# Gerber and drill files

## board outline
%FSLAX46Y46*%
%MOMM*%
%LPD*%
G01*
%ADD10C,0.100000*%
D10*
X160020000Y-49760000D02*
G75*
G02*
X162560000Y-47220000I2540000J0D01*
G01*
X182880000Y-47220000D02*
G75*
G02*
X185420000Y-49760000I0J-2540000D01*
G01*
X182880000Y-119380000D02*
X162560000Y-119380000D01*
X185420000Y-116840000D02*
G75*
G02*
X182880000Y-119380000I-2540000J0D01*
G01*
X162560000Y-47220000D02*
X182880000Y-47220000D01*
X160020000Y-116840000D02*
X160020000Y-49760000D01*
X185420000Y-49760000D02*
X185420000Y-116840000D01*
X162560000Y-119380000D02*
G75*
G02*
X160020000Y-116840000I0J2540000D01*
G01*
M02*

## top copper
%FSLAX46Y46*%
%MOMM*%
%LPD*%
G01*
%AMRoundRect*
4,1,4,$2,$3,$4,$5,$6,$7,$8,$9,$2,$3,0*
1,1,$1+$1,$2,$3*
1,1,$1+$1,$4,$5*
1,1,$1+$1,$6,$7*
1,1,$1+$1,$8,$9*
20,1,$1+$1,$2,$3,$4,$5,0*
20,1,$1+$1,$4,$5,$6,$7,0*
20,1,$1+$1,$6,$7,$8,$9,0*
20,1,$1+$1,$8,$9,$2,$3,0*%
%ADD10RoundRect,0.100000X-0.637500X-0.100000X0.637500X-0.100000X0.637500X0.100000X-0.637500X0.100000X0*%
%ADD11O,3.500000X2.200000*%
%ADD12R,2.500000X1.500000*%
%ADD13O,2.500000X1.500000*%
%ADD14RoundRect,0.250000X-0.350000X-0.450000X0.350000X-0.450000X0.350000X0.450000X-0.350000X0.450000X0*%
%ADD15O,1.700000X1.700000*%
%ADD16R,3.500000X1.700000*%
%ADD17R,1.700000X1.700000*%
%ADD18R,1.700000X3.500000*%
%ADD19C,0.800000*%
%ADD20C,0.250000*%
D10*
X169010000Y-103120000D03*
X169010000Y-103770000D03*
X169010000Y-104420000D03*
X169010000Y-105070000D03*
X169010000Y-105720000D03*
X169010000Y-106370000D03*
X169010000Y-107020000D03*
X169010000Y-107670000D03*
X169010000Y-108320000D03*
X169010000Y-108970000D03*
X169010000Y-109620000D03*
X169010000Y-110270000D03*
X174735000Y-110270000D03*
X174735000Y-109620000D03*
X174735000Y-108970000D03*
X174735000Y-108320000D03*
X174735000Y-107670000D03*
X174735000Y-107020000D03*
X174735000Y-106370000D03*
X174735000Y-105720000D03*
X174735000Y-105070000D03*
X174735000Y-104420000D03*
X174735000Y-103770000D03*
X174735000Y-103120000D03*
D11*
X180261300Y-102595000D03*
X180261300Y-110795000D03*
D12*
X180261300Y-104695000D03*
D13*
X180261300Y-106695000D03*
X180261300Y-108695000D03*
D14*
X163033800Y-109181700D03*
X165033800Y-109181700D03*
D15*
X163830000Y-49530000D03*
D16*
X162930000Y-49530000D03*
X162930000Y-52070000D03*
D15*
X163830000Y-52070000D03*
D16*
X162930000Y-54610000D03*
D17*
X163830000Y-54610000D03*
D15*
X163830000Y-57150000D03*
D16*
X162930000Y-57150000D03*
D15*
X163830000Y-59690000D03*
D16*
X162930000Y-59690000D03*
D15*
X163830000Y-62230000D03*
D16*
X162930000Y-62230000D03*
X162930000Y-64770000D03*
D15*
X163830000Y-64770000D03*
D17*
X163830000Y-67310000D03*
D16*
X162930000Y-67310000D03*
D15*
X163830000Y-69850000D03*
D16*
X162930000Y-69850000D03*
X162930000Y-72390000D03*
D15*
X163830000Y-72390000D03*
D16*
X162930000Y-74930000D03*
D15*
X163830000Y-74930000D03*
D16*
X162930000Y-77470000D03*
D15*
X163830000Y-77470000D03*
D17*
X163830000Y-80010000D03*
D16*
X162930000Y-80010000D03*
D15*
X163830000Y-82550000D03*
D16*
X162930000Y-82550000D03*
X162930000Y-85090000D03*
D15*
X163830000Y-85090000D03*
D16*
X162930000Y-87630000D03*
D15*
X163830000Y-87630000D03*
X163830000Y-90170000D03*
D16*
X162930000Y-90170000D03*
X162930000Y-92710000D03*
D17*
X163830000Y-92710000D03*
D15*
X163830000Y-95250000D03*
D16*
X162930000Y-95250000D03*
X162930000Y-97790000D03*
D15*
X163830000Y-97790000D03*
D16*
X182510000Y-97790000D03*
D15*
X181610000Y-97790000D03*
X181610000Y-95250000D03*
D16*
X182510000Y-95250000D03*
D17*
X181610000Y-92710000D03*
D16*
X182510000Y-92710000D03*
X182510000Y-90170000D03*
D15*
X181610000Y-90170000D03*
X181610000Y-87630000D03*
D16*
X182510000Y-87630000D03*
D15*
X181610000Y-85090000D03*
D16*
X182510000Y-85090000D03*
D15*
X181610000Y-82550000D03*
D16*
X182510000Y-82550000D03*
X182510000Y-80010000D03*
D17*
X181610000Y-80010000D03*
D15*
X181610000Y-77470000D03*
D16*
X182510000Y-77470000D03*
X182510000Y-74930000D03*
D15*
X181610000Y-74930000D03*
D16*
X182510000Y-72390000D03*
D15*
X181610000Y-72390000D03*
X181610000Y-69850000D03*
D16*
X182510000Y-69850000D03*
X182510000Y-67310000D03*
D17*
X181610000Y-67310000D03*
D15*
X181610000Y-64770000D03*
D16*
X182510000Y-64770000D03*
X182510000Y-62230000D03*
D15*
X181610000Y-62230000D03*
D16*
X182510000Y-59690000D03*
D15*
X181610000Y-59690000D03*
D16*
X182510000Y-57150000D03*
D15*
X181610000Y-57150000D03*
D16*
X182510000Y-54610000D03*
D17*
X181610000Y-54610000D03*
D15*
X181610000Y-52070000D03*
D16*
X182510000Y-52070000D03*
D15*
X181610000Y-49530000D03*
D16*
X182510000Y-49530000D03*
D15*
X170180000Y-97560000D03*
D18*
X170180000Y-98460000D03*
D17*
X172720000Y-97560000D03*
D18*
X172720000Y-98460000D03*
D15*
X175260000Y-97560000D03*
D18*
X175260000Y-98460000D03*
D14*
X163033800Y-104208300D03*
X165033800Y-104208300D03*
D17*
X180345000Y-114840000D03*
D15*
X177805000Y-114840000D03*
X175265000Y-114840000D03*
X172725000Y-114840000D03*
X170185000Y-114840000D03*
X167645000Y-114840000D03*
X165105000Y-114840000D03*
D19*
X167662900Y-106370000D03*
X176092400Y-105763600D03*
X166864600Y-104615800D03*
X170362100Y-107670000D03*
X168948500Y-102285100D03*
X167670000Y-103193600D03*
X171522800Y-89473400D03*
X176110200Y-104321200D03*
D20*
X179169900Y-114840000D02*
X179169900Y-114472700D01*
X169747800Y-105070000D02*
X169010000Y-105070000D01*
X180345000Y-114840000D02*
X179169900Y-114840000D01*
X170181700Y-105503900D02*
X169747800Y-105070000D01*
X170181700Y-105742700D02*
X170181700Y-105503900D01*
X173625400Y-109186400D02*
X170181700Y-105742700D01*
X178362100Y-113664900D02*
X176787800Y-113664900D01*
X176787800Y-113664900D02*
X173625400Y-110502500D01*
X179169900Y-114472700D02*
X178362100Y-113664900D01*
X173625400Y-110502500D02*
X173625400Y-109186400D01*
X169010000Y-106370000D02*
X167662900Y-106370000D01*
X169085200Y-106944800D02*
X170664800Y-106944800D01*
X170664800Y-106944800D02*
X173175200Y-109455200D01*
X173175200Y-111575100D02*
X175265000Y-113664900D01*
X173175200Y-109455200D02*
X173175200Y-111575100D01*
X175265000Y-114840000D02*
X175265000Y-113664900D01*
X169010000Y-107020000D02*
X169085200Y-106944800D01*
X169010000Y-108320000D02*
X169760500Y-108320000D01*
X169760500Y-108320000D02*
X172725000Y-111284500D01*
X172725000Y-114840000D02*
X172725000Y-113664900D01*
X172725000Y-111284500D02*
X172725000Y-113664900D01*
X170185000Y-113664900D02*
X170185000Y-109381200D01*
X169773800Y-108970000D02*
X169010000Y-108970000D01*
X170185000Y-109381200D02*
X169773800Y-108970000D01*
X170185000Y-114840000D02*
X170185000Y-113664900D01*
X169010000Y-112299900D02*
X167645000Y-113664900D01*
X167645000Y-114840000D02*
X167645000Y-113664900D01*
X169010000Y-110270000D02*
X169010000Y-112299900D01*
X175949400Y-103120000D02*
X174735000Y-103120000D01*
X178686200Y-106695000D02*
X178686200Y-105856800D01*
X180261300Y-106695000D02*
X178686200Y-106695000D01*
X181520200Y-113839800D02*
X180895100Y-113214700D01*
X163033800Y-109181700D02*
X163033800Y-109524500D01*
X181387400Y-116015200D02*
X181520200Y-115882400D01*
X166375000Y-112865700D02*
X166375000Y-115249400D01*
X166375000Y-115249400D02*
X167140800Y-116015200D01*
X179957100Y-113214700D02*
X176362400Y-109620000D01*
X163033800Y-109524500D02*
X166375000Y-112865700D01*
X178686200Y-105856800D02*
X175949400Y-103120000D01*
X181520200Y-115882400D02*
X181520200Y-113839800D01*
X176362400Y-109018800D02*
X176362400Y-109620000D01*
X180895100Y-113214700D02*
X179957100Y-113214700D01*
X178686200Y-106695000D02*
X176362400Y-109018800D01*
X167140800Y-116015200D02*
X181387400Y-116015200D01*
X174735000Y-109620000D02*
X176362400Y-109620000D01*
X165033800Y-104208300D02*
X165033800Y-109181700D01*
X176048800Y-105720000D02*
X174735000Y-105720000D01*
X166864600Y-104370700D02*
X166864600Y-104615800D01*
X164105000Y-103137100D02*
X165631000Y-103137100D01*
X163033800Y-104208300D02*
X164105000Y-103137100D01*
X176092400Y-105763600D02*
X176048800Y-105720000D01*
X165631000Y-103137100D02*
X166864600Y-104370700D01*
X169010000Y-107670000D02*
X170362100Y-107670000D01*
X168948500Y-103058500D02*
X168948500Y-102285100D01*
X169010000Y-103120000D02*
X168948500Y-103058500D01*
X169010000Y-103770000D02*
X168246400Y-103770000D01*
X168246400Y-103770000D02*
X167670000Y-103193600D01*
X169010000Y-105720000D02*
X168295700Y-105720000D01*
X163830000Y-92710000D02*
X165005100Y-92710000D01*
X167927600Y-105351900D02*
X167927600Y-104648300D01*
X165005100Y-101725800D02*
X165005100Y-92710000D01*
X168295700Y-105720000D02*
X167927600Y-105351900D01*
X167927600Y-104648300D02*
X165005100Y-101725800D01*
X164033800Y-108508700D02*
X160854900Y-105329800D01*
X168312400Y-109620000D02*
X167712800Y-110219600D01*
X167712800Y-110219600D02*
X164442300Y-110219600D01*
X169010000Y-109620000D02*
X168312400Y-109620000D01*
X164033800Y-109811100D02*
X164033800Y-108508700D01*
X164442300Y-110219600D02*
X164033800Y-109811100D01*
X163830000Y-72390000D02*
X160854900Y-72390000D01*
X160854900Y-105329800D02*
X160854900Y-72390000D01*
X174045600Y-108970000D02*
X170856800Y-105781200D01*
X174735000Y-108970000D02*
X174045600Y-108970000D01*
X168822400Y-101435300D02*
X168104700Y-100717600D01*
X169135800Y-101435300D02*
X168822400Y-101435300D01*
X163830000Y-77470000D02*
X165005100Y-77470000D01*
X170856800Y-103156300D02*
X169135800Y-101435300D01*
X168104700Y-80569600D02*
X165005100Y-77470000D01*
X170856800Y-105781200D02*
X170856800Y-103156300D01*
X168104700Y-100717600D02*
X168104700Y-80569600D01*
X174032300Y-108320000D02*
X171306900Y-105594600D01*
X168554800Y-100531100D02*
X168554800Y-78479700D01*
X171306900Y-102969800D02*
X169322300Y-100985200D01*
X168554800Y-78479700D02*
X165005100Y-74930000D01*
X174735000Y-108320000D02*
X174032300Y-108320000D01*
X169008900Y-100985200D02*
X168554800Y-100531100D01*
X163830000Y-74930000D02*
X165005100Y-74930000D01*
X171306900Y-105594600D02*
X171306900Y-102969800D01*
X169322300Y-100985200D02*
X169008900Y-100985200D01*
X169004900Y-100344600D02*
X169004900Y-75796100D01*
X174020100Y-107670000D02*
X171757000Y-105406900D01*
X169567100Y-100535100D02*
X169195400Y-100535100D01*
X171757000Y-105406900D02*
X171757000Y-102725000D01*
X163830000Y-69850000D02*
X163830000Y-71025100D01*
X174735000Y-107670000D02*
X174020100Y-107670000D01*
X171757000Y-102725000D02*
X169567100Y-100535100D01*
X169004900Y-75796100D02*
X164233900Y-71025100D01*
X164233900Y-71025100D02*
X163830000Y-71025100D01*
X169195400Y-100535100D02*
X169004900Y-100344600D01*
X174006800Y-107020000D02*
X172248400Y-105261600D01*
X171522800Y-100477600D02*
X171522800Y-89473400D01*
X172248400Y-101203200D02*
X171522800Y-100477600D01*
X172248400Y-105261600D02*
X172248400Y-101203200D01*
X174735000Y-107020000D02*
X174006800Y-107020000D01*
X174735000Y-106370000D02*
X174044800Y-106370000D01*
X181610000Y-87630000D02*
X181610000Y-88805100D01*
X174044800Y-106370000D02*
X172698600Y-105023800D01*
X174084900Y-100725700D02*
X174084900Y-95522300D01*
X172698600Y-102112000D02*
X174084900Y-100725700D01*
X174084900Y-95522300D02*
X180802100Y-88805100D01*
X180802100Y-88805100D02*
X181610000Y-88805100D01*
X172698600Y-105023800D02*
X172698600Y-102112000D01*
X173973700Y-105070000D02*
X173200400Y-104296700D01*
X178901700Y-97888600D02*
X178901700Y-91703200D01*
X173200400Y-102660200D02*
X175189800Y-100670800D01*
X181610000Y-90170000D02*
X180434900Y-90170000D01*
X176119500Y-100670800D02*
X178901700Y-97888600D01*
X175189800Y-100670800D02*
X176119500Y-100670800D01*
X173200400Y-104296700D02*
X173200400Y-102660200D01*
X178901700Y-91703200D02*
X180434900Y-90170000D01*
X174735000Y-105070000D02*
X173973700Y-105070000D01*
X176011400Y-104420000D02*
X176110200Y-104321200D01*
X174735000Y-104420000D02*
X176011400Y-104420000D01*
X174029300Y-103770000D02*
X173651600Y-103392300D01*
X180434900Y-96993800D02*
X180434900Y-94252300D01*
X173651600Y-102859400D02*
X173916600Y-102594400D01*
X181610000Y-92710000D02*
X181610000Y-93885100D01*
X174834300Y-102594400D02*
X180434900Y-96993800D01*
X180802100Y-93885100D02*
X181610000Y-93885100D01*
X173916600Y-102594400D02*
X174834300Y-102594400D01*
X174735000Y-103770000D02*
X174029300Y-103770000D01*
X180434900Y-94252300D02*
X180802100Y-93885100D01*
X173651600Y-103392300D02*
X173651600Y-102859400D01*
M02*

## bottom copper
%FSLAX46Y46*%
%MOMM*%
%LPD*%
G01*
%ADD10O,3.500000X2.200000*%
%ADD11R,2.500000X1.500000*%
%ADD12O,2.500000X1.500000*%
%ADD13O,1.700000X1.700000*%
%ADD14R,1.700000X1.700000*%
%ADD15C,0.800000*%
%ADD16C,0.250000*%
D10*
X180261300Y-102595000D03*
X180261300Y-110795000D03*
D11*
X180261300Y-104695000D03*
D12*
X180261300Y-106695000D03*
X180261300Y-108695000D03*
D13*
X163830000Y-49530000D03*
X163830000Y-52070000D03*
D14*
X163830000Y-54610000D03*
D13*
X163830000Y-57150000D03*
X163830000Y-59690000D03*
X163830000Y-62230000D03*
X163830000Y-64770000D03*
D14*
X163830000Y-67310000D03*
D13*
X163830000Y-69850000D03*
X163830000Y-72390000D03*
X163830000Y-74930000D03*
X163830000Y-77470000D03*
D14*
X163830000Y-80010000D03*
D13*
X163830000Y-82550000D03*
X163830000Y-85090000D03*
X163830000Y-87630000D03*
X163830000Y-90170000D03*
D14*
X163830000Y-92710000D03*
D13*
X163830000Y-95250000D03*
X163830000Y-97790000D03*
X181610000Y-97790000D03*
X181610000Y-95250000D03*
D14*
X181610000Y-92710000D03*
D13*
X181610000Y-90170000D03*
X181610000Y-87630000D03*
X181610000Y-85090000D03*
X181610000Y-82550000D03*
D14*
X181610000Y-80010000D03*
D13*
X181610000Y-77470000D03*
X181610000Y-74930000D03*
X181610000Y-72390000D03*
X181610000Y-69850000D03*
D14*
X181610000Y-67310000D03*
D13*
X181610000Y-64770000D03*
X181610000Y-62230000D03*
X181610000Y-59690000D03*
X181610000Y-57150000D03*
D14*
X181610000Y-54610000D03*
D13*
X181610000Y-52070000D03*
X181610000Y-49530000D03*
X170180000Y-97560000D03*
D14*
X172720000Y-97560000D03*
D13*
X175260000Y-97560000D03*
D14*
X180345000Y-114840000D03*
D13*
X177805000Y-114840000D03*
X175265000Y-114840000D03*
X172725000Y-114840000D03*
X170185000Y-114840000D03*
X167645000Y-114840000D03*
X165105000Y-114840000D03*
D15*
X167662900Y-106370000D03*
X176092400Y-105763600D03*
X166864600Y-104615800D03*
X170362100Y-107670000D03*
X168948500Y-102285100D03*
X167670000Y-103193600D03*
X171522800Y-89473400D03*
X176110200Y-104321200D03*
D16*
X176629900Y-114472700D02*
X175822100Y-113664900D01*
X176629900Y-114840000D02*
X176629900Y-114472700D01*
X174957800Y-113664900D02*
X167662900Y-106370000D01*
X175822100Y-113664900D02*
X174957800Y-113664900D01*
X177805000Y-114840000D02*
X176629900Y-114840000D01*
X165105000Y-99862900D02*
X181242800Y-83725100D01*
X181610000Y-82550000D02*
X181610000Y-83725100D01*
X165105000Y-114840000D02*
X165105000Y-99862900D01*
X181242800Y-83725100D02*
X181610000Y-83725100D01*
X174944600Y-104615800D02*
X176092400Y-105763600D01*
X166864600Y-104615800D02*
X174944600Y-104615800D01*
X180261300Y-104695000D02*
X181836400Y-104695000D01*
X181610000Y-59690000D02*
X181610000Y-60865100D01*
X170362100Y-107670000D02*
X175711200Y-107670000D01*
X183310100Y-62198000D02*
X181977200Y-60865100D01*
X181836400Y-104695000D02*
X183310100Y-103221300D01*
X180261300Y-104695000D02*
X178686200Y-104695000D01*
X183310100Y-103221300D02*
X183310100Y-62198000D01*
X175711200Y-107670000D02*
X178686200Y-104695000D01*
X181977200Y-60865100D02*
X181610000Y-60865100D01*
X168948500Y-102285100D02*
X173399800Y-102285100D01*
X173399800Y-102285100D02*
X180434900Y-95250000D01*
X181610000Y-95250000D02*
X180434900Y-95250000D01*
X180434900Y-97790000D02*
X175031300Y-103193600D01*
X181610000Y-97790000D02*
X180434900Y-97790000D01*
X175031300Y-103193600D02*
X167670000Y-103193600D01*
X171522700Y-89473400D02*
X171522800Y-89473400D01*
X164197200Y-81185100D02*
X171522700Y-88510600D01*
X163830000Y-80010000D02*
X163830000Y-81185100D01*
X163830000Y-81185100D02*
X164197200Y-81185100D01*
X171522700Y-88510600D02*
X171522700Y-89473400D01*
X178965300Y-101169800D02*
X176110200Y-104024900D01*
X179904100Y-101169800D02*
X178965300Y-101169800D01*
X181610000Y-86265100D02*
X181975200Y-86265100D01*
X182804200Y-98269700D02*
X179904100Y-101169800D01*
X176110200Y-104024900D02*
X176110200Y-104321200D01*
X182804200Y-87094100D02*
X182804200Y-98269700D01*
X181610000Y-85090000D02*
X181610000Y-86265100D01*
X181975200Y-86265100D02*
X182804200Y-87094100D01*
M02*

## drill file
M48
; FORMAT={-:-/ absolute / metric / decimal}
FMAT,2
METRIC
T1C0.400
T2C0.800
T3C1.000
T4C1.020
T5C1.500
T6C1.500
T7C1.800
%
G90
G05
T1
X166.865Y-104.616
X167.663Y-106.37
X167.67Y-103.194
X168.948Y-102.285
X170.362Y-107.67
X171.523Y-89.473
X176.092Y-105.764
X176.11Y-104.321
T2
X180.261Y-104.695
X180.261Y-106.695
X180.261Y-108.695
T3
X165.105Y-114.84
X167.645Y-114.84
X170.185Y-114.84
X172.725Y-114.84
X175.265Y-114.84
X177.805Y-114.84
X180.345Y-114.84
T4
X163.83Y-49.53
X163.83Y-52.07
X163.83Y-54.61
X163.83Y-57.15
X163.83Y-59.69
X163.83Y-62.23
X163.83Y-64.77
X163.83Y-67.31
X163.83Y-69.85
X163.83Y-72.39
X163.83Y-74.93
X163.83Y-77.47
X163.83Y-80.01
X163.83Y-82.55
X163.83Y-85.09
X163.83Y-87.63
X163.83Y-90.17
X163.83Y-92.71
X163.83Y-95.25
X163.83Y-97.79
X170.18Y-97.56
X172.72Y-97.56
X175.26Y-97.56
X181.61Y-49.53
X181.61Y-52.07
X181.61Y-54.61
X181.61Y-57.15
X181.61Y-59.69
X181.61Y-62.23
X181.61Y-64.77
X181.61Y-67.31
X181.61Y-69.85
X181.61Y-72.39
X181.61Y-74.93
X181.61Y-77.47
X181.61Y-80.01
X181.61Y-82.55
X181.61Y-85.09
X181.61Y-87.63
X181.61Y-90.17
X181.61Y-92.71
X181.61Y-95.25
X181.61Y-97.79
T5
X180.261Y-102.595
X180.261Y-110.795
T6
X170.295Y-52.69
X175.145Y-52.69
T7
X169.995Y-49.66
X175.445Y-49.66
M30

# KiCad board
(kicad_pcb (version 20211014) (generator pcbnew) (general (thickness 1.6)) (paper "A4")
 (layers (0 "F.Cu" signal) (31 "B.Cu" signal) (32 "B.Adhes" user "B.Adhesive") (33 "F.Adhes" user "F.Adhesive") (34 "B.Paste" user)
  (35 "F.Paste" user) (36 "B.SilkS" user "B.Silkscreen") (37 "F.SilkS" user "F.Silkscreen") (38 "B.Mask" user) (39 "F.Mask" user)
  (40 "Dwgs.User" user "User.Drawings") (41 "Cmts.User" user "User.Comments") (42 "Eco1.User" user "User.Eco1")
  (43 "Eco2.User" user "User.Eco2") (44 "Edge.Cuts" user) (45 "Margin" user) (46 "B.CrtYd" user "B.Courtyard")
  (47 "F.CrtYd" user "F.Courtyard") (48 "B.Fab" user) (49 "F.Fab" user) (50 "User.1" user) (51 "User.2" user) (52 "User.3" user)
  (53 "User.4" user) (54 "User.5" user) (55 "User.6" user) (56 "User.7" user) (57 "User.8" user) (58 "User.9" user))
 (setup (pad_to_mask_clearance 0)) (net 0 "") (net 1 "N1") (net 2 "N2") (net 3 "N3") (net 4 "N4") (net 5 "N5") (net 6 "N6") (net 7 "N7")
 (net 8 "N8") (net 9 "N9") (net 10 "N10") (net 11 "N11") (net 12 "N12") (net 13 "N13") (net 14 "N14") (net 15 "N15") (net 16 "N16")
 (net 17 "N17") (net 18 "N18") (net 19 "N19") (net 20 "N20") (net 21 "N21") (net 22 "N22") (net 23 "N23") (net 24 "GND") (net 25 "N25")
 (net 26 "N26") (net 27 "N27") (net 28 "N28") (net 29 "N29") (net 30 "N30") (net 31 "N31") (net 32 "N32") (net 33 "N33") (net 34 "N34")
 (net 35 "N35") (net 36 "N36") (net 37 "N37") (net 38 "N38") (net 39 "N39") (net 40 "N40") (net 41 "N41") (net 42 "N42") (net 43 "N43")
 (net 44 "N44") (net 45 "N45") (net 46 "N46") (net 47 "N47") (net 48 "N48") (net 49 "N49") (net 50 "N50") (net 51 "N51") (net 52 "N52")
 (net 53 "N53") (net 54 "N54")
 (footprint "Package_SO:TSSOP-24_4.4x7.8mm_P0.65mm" (layer "F.Cu") (at 171.8725 106.695)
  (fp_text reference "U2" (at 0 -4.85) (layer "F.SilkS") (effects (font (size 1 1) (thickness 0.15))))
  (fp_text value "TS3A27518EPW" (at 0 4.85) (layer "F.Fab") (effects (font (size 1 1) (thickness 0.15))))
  (pad "1" smd roundrect (at -2.8625 -3.575) (size 1.475 0.4) (layers "F.Cu" "F.Paste" "F.Mask") (roundrect_rratio 0.25) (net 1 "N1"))
  (pad "2" smd roundrect (at -2.8625 -2.925) (size 1.475 0.4) (layers "F.Cu" "F.Paste" "F.Mask") (roundrect_rratio 0.25) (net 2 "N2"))
  (pad "3" smd roundrect (at -2.8625 -2.275) (size 1.475 0.4) (layers "F.Cu" "F.Paste" "F.Mask") (roundrect_rratio 0.25) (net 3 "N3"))
  (pad "4" smd roundrect (at -2.8625 -1.625) (size 1.475 0.4) (layers "F.Cu" "F.Paste" "F.Mask") (roundrect_rratio 0.25) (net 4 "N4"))
  (pad "5" smd roundrect (at -2.8625 -0.975) (size 1.475 0.4) (layers "F.Cu" "F.Paste" "F.Mask") (roundrect_rratio 0.25) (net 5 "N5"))
  (pad "6" smd roundrect (at -2.8625 -0.325) (size 1.475 0.4) (layers "F.Cu" "F.Paste" "F.Mask") (roundrect_rratio 0.25) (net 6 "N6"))
  (pad "7" smd roundrect (at -2.8625 0.325) (size 1.475 0.4) (layers "F.Cu" "F.Paste" "F.Mask") (roundrect_rratio 0.25) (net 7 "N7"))
  (pad "8" smd roundrect (at -2.8625 0.975) (size 1.475 0.4) (layers "F.Cu" "F.Paste" "F.Mask") (roundrect_rratio 0.25) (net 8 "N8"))
  (pad "9" smd roundrect (at -2.8625 1.625) (size 1.475 0.4) (layers "F.Cu" "F.Paste" "F.Mask") (roundrect_rratio 0.25) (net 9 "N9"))
  (pad "10" smd roundrect (at -2.8625 2.275) (size 1.475 0.4) (layers "F.Cu" "F.Paste" "F.Mask") (roundrect_rratio 0.25) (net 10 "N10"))
  (pad "11" smd roundrect (at -2.8625 2.925) (size 1.475 0.4) (layers "F.Cu" "F.Paste" "F.Mask") (roundrect_rratio 0.25) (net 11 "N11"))
  (pad "12" smd roundrect (at -2.8625 3.575) (size 1.475 0.4) (layers "F.Cu" "F.Paste" "F.Mask") (roundrect_rratio 0.25) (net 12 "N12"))
  (pad "13" smd roundrect (at 2.8625 3.575) (size 1.475 0.4) (layers "F.Cu" "F.Paste" "F.Mask") (roundrect_rratio 0.25) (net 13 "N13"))
  (pad "14" smd roundrect (at 2.8625 2.925) (size 1.475 0.4) (layers "F.Cu" "F.Paste" "F.Mask") (roundrect_rratio 0.25) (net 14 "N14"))
  (pad "15" smd roundrect (at 2.8625 2.275) (size 1.475 0.4) (layers "F.Cu" "F.Paste" "F.Mask") (roundrect_rratio 0.25) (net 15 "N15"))
  (pad "16" smd roundrect (at 2.8625 1.625) (size 1.475 0.4) (layers "F.Cu" "F.Paste" "F.Mask") (roundrect_rratio 0.25) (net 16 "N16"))
  (pad "17" smd roundrect (at 2.8625 0.975) (size 1.475 0.4) (layers "F.Cu" "F.Paste" "F.Mask") (roundrect_rratio 0.25) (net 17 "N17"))
  (pad "18" smd roundrect (at 2.8625 0.325) (size 1.475 0.4) (layers "F.Cu" "F.Paste" "F.Mask") (roundrect_rratio 0.25) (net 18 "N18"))
  (pad "19" smd roundrect (at 2.8625 -0.325) (size 1.475 0.4) (layers "F.Cu" "F.Paste" "F.Mask") (roundrect_rratio 0.25) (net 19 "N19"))
  (pad "20" smd roundrect (at 2.8625 -0.975) (size 1.475 0.4) (layers "F.Cu" "F.Paste" "F.Mask") (roundrect_rratio 0.25) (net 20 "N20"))
  (pad "21" smd roundrect (at 2.8625 -1.625) (size 1.475 0.4) (layers "F.Cu" "F.Paste" "F.Mask") (roundrect_rratio 0.25) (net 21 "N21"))
  (pad "22" smd roundrect (at 2.8625 -2.275) (size 1.475 0.4) (layers "F.Cu" "F.Paste" "F.Mask") (roundrect_rratio 0.25) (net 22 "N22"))
  (pad "23" smd roundrect (at 2.8625 -2.925) (size 1.475 0.4) (layers "F.Cu" "F.Paste" "F.Mask") (roundrect_rratio 0.25) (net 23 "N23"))
  (pad "24" smd roundrect (at 2.8625 -3.575) (size 1.475 0.4) (layers "F.Cu" "F.Paste" "F.Mask") (roundrect_rratio 0.25) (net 14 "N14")))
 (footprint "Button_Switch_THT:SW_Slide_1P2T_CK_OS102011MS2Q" (layer "F.Cu") (at 180.2613 104.695 -90)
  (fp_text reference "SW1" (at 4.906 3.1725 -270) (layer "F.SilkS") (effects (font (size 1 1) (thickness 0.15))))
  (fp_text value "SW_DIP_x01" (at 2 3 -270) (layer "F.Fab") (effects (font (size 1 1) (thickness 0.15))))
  (pad "" thru_hole oval (at -2.1 0 270) (size 2.2 3.5) (drill 1.5) (layers *.Cu *.Mask))
  (pad "" thru_hole oval (at 6.1 0 270) (size 2.2 3.5) (drill 1.5) (layers *.Cu *.Mask))
  (pad "1" thru_hole rect (at 0 0 270) (size 1.5 2.5) (drill 0.8) (layers *.Cu *.Mask) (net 8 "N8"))
  (pad "2" thru_hole oval (at 2 0 270) (size 1.5 2.5) (drill 0.8) (layers *.Cu *.Mask) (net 14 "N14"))
  (pad "3" thru_hole oval (at 4 0 270) (size 1.5 2.5) (drill 0.8) (layers *.Cu *.Mask)))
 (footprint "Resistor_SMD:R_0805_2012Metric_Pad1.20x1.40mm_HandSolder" (layer "F.Cu") (at 164.0338 109.1817)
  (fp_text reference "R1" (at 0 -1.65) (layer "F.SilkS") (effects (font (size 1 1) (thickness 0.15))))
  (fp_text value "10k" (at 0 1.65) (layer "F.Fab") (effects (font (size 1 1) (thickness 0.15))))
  (pad "1" smd roundrect (at -1 0) (size 1.2 1.4) (layers "F.Cu" "F.Paste" "F.Mask") (roundrect_rratio 0.208333) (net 14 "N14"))
  (pad "2" smd roundrect (at 1 0) (size 1.2 1.4) (layers "F.Cu" "F.Paste" "F.Mask") (roundrect_rratio 0.208333) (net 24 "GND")))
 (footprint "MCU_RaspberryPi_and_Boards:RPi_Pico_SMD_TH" (layer "F.Cu") (at 172.72 73.66)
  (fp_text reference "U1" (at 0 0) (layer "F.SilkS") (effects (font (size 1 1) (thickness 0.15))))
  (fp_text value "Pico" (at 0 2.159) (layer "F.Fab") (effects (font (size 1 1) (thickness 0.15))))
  (pad "" np_thru_hole oval (at 2.425 -20.97) (size 1.5 1.5) (drill 1.5) (layers *.Cu *.Mask))
  (pad "" np_thru_hole oval (at 2.725 -24) (size 1.8 1.8) (drill 1.8) (layers *.Cu *.Mask))
  (pad "" np_thru_hole oval (at -2.725 -24) (size 1.8 1.8) (drill 1.8) (layers *.Cu *.Mask))
  (pad "" np_thru_hole oval (at -2.425 -20.97) (size 1.5 1.5) (drill 1.5) (layers *.Cu *.Mask))
  (pad "1" thru_hole oval (at -8.89 -24.13) (size 1.7 1.7) (drill 1.02) (layers *.Cu *.Mask) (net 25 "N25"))
  (pad "1" smd rect (at -8.89 -24.13) (size 3.5 1.7) (drill (offset -0.9 0)) (layers "F.Cu" "F.Mask") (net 25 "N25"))
  (pad "2" smd rect (at -8.89 -21.59) (size 3.5 1.7) (drill (offset -0.9 0)) (layers "F.Cu" "F.Mask") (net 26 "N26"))
  (pad "2" thru_hole oval (at -8.89 -21.59) (size 1.7 1.7) (drill 1.02) (layers *.Cu *.Mask) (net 26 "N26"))
  (pad "3" smd rect (at -8.89 -19.05) (size 3.5 1.7) (drill (offset -0.9 0)) (layers "F.Cu" "F.Mask") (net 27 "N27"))
  (pad "3" thru_hole rect (at -8.89 -19.05) (size 1.7 1.7) (drill 1.02) (layers *.Cu *.Mask) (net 27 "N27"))
  (pad "4" thru_hole oval (at -8.89 -16.51) (size 1.7 1.7) (drill 1.02) (layers *.Cu *.Mask) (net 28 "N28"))
  (pad "4" smd rect (at -8.89 -16.51) (size 3.5 1.7) (drill (offset -0.9 0)) (layers "F.Cu" "F.Mask") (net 28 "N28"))
  (pad "5" thru_hole oval (at -8.89 -13.97) (size 1.7 1.7) (drill 1.02) (layers *.Cu *.Mask) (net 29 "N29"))
  (pad "5" smd rect (at -8.89 -13.97) (size 3.5 1.7) (drill (offset -0.9 0)) (layers "F.Cu" "F.Mask") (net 29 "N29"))
  (pad "6" thru_hole oval (at -8.89 -11.43) (size 1.7 1.7) (drill 1.02) (layers *.Cu *.Mask) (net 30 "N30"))
  (pad "6" smd rect (at -8.89 -11.43) (size 3.5 1.7) (drill (offset -0.9 0)) (layers "F.Cu" "F.Mask") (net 30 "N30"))
  (pad "7" smd rect (at -8.89 -8.89) (size 3.5 1.7) (drill (offset -0.9 0)) (layers "F.Cu" "F.Mask") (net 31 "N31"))
  (pad "7" thru_hole oval (at -8.89 -8.89) (size 1.7 1.7) (drill 1.02) (layers *.Cu *.Mask) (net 31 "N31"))
  (pad "8" thru_hole rect (at -8.89 -6.35) (size 1.7 1.7) (drill 1.02) (layers *.Cu *.Mask) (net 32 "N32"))
  (pad "8" smd rect (at -8.89 -6.35) (size 3.5 1.7) (drill (offset -0.9 0)) (layers "F.Cu" "F.Mask") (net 32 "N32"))
  (pad "9" thru_hole oval (at -8.89 -3.81) (size 1.7 1.7) (drill 1.02) (layers *.Cu *.Mask) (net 17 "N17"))
  (pad "9" smd rect (at -8.89 -3.81) (size 3.5 1.7) (drill (offset -0.9 0)) (layers "F.Cu" "F.Mask") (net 17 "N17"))
  (pad "10" smd rect (at -8.89 -1.27) (size 3.5 1.7) (drill (offset -0.9 0)) (layers "F.Cu" "F.Mask") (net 11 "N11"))
  (pad "10" thru_hole oval (at -8.89 -1.27) (size 1.7 1.7) (drill 1.02) (layers *.Cu *.Mask) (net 11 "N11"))
  (pad "11" smd rect (at -8.89 1.27) (size 3.5 1.7) (drill (offset -0.9 0)) (layers "F.Cu" "F.Mask") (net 16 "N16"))
  (pad "11" thru_hole oval (at -8.89 1.27) (size 1.7 1.7) (drill 1.02) (layers *.Cu *.Mask) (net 16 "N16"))
  (pad "12" smd rect (at -8.89 3.81) (size 3.5 1.7) (drill (offset -0.9 0)) (layers "F.Cu" "F.Mask") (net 15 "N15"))
  (pad "12" thru_hole oval (at -8.89 3.81) (size 1.7 1.7) (drill 1.02) (layers *.Cu *.Mask) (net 15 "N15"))
  (pad "13" thru_hole rect (at -8.89 6.35) (size 1.7 1.7) (drill 1.02) (layers *.Cu *.Mask) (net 18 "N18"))
  (pad "13" smd rect (at -8.89 6.35) (size 3.5 1.7) (drill (offset -0.9 0)) (layers "F.Cu" "F.Mask") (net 18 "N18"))
  (pad "14" thru_hole oval (at -8.89 8.89) (size 1.7 1.7) (drill 1.02) (layers *.Cu *.Mask) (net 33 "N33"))
  (pad "14" smd rect (at -8.89 8.89) (size 3.5 1.7) (drill (offset -0.9 0)) (layers "F.Cu" "F.Mask") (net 33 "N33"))
  (pad "15" smd rect (at -8.89 11.43) (size 3.5 1.7) (drill (offset -0.9 0)) (layers "F.Cu" "F.Mask") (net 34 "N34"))
  (pad "15" thru_hole oval (at -8.89 11.43) (size 1.7 1.7) (drill 1.02) (layers *.Cu *.Mask) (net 34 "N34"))
  (pad "16" smd rect (at -8.89 13.97) (size 3.5 1.7) (drill (offset -0.9 0)) (layers "F.Cu" "F.Mask") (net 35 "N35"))
  (pad "16" thru_hole oval (at -8.89 13.97) (size 1.7 1.7) (drill 1.02) (layers *.Cu *.Mask) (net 35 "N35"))
  (pad "17" thru_hole oval (at -8.89 16.51) (size 1.7 1.7) (drill 1.02) (layers *.Cu *.Mask) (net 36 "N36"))
  (pad "17" smd rect (at -8.89 16.51) (size 3.5 1.7) (drill (offset -0.9 0)) (layers "F.Cu" "F.Mask") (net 36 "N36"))
  (pad "18" smd rect (at -8.89 19.05) (size 3.5 1.7) (drill (offset -0.9 0)) (layers "F.Cu" "F.Mask") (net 5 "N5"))
  (pad "18" thru_hole rect (at -8.89 19.05) (size 1.7 1.7) (drill 1.02) (layers *.Cu *.Mask) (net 5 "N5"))
  (pad "19" thru_hole oval (at -8.89 21.59) (size 1.7 1.7) (drill 1.02) (layers *.Cu *.Mask) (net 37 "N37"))
  (pad "19" smd rect (at -8.89 21.59) (size 3.5 1.7) (drill (offset -0.9 0)) (layers "F.Cu" "F.Mask") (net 37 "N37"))
  (pad "20" smd rect (at -8.89 24.13) (size 3.5 1.7) (drill (offset -0.9 0)) (layers "F.Cu" "F.Mask") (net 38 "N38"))
  (pad "20" thru_hole oval (at -8.89 24.13) (size 1.7 1.7) (drill 1.02) (layers *.Cu *.Mask) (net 38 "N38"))
  (pad "21" smd rect (at 8.89 24.13) (size 3.5 1.7) (drill (offset 0.9 0)) (layers "F.Cu" "F.Mask") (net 2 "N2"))
  (pad "21" thru_hole oval (at 8.89 24.13) (size 1.7 1.7) (drill 1.02) (layers *.Cu *.Mask) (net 2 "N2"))
  (pad "22" thru_hole oval (at 8.89 21.59) (size 1.7 1.7) (drill 1.02) (layers *.Cu *.Mask) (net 1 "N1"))
  (pad "22" smd rect (at 8.89 21.59) (size 3.5 1.7) (drill (offset 0.9 0)) (layers "F.Cu" "F.Mask") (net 1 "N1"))
  (pad "23" thru_hole rect (at 8.89 19.05) (size 1.7 1.7) (drill 1.02) (layers *.Cu *.Mask) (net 23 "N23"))
  (pad "23" smd rect (at 8.89 19.05) (size 3.5 1.7) (drill (offset 0.9 0)) (layers "F.Cu" "F.Mask") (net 23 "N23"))
  (pad "24" smd rect (at 8.89 16.51) (size 3.5 1.7) (drill (offset 0.9 0)) (layers "F.Cu" "F.Mask") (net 21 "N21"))
  (pad "24" thru_hole oval (at 8.89 16.51) (size 1.7 1.7) (drill 1.02) (layers *.Cu *.Mask) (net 21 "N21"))
  (pad "25" thru_hole oval (at 8.89 13.97) (size 1.7 1.7) (drill 1.02) (layers *.Cu *.Mask) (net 19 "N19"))
  (pad "25" smd rect (at 8.89 13.97) (size 3.5 1.7) (drill (offset 0.9 0)) (layers "F.Cu" "F.Mask") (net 19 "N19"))
  (pad "26" thru_hole oval (at 8.89 11.43) (size 1.7 1.7) (drill 1.02) (layers *.Cu *.Mask) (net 22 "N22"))
  (pad "26" smd rect (at 8.89 11.43) (size 3.5 1.7) (drill (offset 0.9 0)) (layers "F.Cu" "F.Mask") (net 22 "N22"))
  (pad "27" thru_hole oval (at 8.89 8.89) (size 1.7 1.7) (drill 1.02) (layers *.Cu *.Mask) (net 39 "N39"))
  (pad "27" smd rect (at 8.89 8.89) (size 3.5 1.7) (drill (offset 0.9 0)) (layers "F.Cu" "F.Mask") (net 39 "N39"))
  (pad "28" smd rect (at 8.89 6.35) (size 3.5 1.7) (drill (offset 0.9 0)) (layers "F.Cu" "F.Mask") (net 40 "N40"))
  (pad "28" thru_hole rect (at 8.89 6.35) (size 1.7 1.7) (drill 1.02) (layers *.Cu *.Mask) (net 40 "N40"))
  (pad "29" thru_hole oval (at 8.89 3.81) (size 1.7 1.7) (drill 1.02) (layers *.Cu *.Mask) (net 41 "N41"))
  (pad "29" smd rect (at 8.89 3.81) (size 3.5 1.7) (drill (offset 0.9 0)) (layers "F.Cu" "F.Mask") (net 41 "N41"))
  (pad "30" smd rect (at 8.89 1.27) (size 3.5 1.7) (drill (offset 0.9 0)) (layers "F.Cu" "F.Mask") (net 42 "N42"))
  (pad "30" thru_hole oval (at 8.89 1.27) (size 1.7 1.7) (drill 1.02) (layers *.Cu *.Mask) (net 42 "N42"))
  (pad "31" smd rect (at 8.89 -1.27) (size 3.5 1.7) (drill (offset 0.9 0)) (layers "F.Cu" "F.Mask") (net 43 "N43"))
  (pad "31" thru_hole oval (at 8.89 -1.27) (size 1.7 1.7) (drill 1.02) (layers *.Cu *.Mask) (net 43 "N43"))
  (pad "32" thru_hole oval (at 8.89 -3.81) (size 1.7 1.7) (drill 1.02) (layers *.Cu *.Mask) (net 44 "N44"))
  (pad "32" smd rect (at 8.89 -3.81) (size 3.5 1.7) (drill (offset 0.9 0)) (layers "F.Cu" "F.Mask") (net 44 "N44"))
  (pad "33" smd rect (at 8.89 -6.35) (size 3.5 1.7) (drill (offset 0.9 0)) (layers "F.Cu" "F.Mask") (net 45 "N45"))
  (pad "33" thru_hole rect (at 8.89 -6.35) (size 1.7 1.7) (drill 1.02) (layers *.Cu *.Mask) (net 45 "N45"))
  (pad "34" thru_hole oval (at 8.89 -8.89) (size 1.7 1.7) (drill 1.02) (layers *.Cu *.Mask) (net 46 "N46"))
  (pad "34" smd rect (at 8.89 -8.89) (size 3.5 1.7) (drill (offset 0.9 0)) (layers "F.Cu" "F.Mask") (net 46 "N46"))
  (pad "35" smd rect (at 8.89 -11.43) (size 3.5 1.7) (drill (offset 0.9 0)) (layers "F.Cu" "F.Mask") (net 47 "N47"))
  (pad "35" thru_hole oval (at 8.89 -11.43) (size 1.7 1.7) (drill 1.02) (layers *.Cu *.Mask) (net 47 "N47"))
  (pad "36" smd rect (at 8.89 -13.97) (size 3.5 1.7) (drill (offset 0.9 0)) (layers "F.Cu" "F.Mask") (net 8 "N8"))
  (pad "36" thru_hole oval (at 8.89 -13.97) (size 1.7 1.7) (drill 1.02) (layers *.Cu *.Mask) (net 8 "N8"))
  (pad "37" smd rect (at 8.89 -16.51) (size 3.5 1.7) (drill (offset 0.9 0)) (layers "F.Cu" "F.Mask") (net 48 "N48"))
  (pad "37" thru_hole oval (at 8.89 -16.51) (size 1.7 1.7) (drill 1.02) (layers *.Cu *.Mask) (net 48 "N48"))
  (pad "38" smd rect (at 8.89 -19.05) (size 3.5 1.7) (drill (offset 0.9 0)) (layers "F.Cu" "F.Mask") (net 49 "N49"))
  (pad "38" thru_hole rect (at 8.89 -19.05) (size 1.7 1.7) (drill 1.02) (layers *.Cu *.Mask) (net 49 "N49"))
  (pad "39" thru_hole oval (at 8.89 -21.59) (size 1.7 1.7) (drill 1.02) (layers *.Cu *.Mask) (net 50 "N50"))
  (pad "39" smd rect (at 8.89 -21.59) (size 3.5 1.7) (drill (offset 0.9 0)) (layers "F.Cu" "F.Mask") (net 50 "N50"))
  (pad "40" thru_hole oval (at 8.89 -24.13) (size 1.7 1.7) (drill 1.02) (layers *.Cu *.Mask) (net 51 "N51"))
  (pad "40" smd rect (at 8.89 -24.13) (size 3.5 1.7) (drill (offset 0.9 0)) (layers "F.Cu" "F.Mask") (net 51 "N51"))
  (pad "41" thru_hole oval (at -2.54 23.9) (size 1.7 1.7) (drill 1.02) (layers *.Cu *.Mask) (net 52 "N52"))
  (pad "41" smd rect (at -2.54 23.9 90) (size 3.5 1.7) (drill (offset -0.9 0)) (layers "F.Cu" "F.Mask") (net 52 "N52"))
  (pad "42" thru_hole rect (at 0 23.9) (size 1.7 1.7) (drill 1.02) (layers *.Cu *.Mask) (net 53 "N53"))
  (pad "42" smd rect (at 0 23.9 90) (size 3.5 1.7) (drill (offset -0.9 0)) (layers "F.Cu" "F.Mask") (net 53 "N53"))
  (pad "43" thru_hole oval (at 2.54 23.9) (size 1.7 1.7) (drill 1.02) (layers *.Cu *.Mask) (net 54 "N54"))
  (pad "43" smd rect (at 2.54 23.9 90) (size 3.5 1.7) (drill (offset -0.9 0)) (layers "F.Cu" "F.Mask") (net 54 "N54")))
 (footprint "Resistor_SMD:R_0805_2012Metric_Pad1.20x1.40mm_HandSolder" (layer "F.Cu") (at 164.0338 104.2083)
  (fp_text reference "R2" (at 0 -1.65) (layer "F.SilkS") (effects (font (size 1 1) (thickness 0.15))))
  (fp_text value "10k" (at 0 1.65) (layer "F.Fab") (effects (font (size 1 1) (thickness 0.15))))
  (pad "1" smd roundrect (at -1 0) (size 1.2 1.4) (layers "F.Cu" "F.Paste" "F.Mask") (roundrect_rratio 0.208333) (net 20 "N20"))
  (pad "2" smd roundrect (at 1 0) (size 1.2 1.4) (layers "F.Cu" "F.Paste" "F.Mask") (roundrect_rratio 0.208333) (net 24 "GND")))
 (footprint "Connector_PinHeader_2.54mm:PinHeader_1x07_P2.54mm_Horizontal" (layer "F.Cu") (at 180.345 114.84 -90)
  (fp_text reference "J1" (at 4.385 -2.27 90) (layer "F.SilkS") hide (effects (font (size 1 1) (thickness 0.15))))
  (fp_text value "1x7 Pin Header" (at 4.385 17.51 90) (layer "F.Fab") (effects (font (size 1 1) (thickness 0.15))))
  (pad "1" thru_hole rect (at 0 0 270) (size 1.7 1.7) (drill 1) (layers *.Cu *.Mask) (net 4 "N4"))
  (pad "2" thru_hole oval (at 0 2.54 270) (size 1.7 1.7) (drill 1) (layers *.Cu *.Mask) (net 6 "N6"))
  (pad "3" thru_hole oval (at 0 5.08 270) (size 1.7 1.7) (drill 1) (layers *.Cu *.Mask) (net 7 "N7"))
  (pad "4" thru_hole oval (at 0 7.62 270) (size 1.7 1.7) (drill 1) (layers *.Cu *.Mask) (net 9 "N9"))
  (pad "5" thru_hole oval (at 0 10.16 270) (size 1.7 1.7) (drill 1) (layers *.Cu *.Mask) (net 10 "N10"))
  (pad "6" thru_hole oval (at 0 12.7 270) (size 1.7 1.7) (drill 1) (layers *.Cu *.Mask) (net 12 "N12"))
  (pad "7" thru_hole oval (at 0 15.24 270) (size 1.7 1.7) (drill 1) (layers *.Cu *.Mask) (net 39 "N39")))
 (gr_arc (start 160.02 49.76) (mid 160.763949 47.963949) (end 162.56 47.22) (layer "Edge.Cuts") (width 0.1))
 (gr_arc (start 182.88 47.22) (mid 184.676051 47.963949) (end 185.42 49.76) (layer "Edge.Cuts") (width 0.1))
 (gr_line (start 182.88 119.38) (end 162.56 119.38) (layer "Edge.Cuts") (width 0.1))
 (gr_arc (start 185.42 116.84) (mid 184.676051 118.636051) (end 182.88 119.38) (layer "Edge.Cuts") (width 0.1))
 (gr_line (start 162.56 47.22) (end 182.88 47.22) (layer "Edge.Cuts") (width 0.1))
 (gr_line (start 160.02 116.84) (end 160.02 49.76) (layer "Edge.Cuts") (width 0.1))
 (gr_line (start 185.42 49.76) (end 185.42 116.84) (layer "Edge.Cuts") (width 0.1))
 (gr_arc (start 162.56 119.38) (mid 160.763949 118.636051) (end 160.02 116.84) (layer "Edge.Cuts") (width 0.1))
 (segment (start 179.1699 114.84) (end 179.1699 114.4727) (width 0.25) (layer "F.Cu") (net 4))
 (segment (start 169.7478 105.07) (end 169.01 105.07) (width 0.25) (layer "F.Cu") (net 4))
 (segment (start 180.345 114.84) (end 179.1699 114.84) (width 0.25) (layer "F.Cu") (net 4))
 (segment (start 170.1817 105.5039) (end 169.7478 105.07) (width 0.25) (layer "F.Cu") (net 4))
 (segment (start 170.1817 105.7427) (end 170.1817 105.5039) (width 0.25) (layer "F.Cu") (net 4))
 (segment (start 173.6254 109.1864) (end 170.1817 105.7427) (width 0.25) (layer "F.Cu") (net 4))
 (segment (start 178.3621 113.6649) (end 176.7878 113.6649) (width 0.25) (layer "F.Cu") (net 4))
 (segment (start 176.7878 113.6649) (end 173.6254 110.5025) (width 0.25) (layer "F.Cu") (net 4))
 (segment (start 179.1699 114.4727) (end 178.3621 113.6649) (width 0.25) (layer "F.Cu") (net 4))
 (segment (start 173.6254 110.5025) (end 173.6254 109.1864) (width 0.25) (layer "F.Cu") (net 4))
 (segment (start 169.01 106.37) (end 167.6629 106.37) (width 0.25) (layer "F.Cu") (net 6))
 (via (at 167.6629 106.37) (size 0.8) (drill 0.4) (layers "F.Cu" "B.Cu") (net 6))
 (segment (start 176.6299 114.4727) (end 175.8221 113.6649) (width 0.25) (layer "B.Cu") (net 6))
 (segment (start 176.6299 114.84) (end 176.6299 114.4727) (width 0.25) (layer "B.Cu") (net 6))
 (segment (start 174.9578 113.6649) (end 167.6629 106.37) (width 0.25) (layer "B.Cu") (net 6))
 (segment (start 175.8221 113.6649) (end 174.9578 113.6649) (width 0.25) (layer "B.Cu") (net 6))
 (segment (start 177.805 114.84) (end 176.6299 114.84) (width 0.25) (layer "B.Cu") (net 6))
 (segment (start 169.0852 106.9448) (end 170.6648 106.9448) (width 0.25) (layer "F.Cu") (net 7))
 (segment (start 170.6648 106.9448) (end 173.1752 109.4552) (width 0.25) (layer "F.Cu") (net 7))
 (segment (start 173.1752 111.5751) (end 175.265 113.6649) (width 0.25) (layer "F.Cu") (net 7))
 (segment (start 173.1752 109.4552) (end 173.1752 111.5751) (width 0.25) (layer "F.Cu") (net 7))
 (segment (start 175.265 114.84) (end 175.265 113.6649) (width 0.25) (layer "F.Cu") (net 7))
 (segment (start 169.01 107.02) (end 169.0852 106.9448) (width 0.25) (layer "F.Cu") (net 7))
 (segment (start 169.01 108.32) (end 169.7605 108.32) (width 0.25) (layer "F.Cu") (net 9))
 (segment (start 169.7605 108.32) (end 172.725 111.2845) (width 0.25) (layer "F.Cu") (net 9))
 (segment (start 172.725 114.84) (end 172.725 113.6649) (width 0.25) (layer "F.Cu") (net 9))
 (segment (start 172.725 111.2845) (end 172.725 113.6649) (width 0.25) (layer "F.Cu") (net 9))
 (segment (start 170.185 113.6649) (end 170.185 109.3812) (width 0.25) (layer "F.Cu") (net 10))
 (segment (start 169.7738 108.97) (end 169.01 108.97) (width 0.25) (layer "F.Cu") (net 10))
 (segment (start 170.185 109.3812) (end 169.7738 108.97) (width 0.25) (layer "F.Cu") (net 10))
 (segment (start 170.185 114.84) (end 170.185 113.6649) (width 0.25) (layer "F.Cu") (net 10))
 (segment (start 169.01 112.2999) (end 167.645 113.6649) (width 0.25) (layer "F.Cu") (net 12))
 (segment (start 167.645 114.84) (end 167.645 113.6649) (width 0.25) (layer "F.Cu") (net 12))
 (segment (start 169.01 110.27) (end 169.01 112.2999) (width 0.25) (layer "F.Cu") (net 12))
 (segment (start 165.105 99.8629) (end 181.2428 83.7251) (width 0.25) (layer "B.Cu") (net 39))
 (segment (start 181.61 82.55) (end 181.61 83.7251) (width 0.25) (layer "B.Cu") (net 39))
 (segment (start 165.105 114.84) (end 165.105 99.8629) (width 0.25) (layer "B.Cu") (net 39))
 (segment (start 181.2428 83.7251) (end 181.61 83.7251) (width 0.25) (layer "B.Cu") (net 39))
 (segment (start 175.9494 103.12) (end 174.735 103.12) (width 0.25) (layer "F.Cu") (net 14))
 (segment (start 178.6862 106.695) (end 178.6862 105.8568) (width 0.25) (layer "F.Cu") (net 14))
 (segment (start 180.2613 106.695) (end 178.6862 106.695) (width 0.25) (layer "F.Cu") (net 14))
 (segment (start 181.5202 113.8398) (end 180.8951 113.2147) (width 0.25) (layer "F.Cu") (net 14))
 (segment (start 163.0338 109.1817) (end 163.0338 109.5245) (width 0.25) (layer "F.Cu") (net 14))
 (segment (start 181.3874 116.0152) (end 181.5202 115.8824) (width 0.25) (layer "F.Cu") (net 14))
 (segment (start 166.375 112.8657) (end 166.375 115.2494) (width 0.25) (layer "F.Cu") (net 14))
 (segment (start 166.375 115.2494) (end 167.1408 116.0152) (width 0.25) (layer "F.Cu") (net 14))
 (segment (start 179.9571 113.2147) (end 176.3624 109.62) (width 0.25) (layer "F.Cu") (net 14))
 (segment (start 163.0338 109.5245) (end 166.375 112.8657) (width 0.25) (layer "F.Cu") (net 14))
 (segment (start 178.6862 105.8568) (end 175.9494 103.12) (width 0.25) (layer "F.Cu") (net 14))
 (segment (start 181.5202 115.8824) (end 181.5202 113.8398) (width 0.25) (layer "F.Cu") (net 14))
 (segment (start 176.3624 109.0188) (end 176.3624 109.62) (width 0.25) (layer "F.Cu") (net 14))
 (segment (start 180.8951 113.2147) (end 179.9571 113.2147) (width 0.25) (layer "F.Cu") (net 14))
 (segment (start 178.6862 106.695) (end 176.3624 109.0188) (width 0.25) (layer "F.Cu") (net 14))
 (segment (start 167.1408 116.0152) (end 181.3874 116.0152) (width 0.25) (layer "F.Cu") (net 14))
 (segment (start 174.735 109.62) (end 176.3624 109.62) (width 0.25) (layer "F.Cu") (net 14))
 (segment (start 165.0338 104.2083) (end 165.0338 109.1817) (width 0.25) (layer "F.Cu") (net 24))
 (segment (start 176.0488 105.72) (end 174.735 105.72) (width 0.25) (layer "F.Cu") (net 20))
 (segment (start 166.8646 104.3707) (end 166.8646 104.6158) (width 0.25) (layer "F.Cu") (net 20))
 (segment (start 164.105 103.1371) (end 165.631 103.1371) (width 0.25) (layer "F.Cu") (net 20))
 (segment (start 163.0338 104.2083) (end 164.105 103.1371) (width 0.25) (layer "F.Cu") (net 20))
 (segment (start 176.0924 105.7636) (end 176.0488 105.72) (width 0.25) (layer "F.Cu") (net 20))
 (segment (start 165.631 103.1371) (end 166.8646 104.3707) (width 0.25) (layer "F.Cu") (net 20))
 (via (at 176.0924 105.7636) (size 0.8) (drill 0.4) (layers "F.Cu" "B.Cu") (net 20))
 (via (at 166.8646 104.6158) (size 0.8) (drill 0.4) (layers "F.Cu" "B.Cu") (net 20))
 (segment (start 174.9446 104.6158) (end 176.0924 105.7636) (width 0.25) (layer "B.Cu") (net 20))
 (segment (start 166.8646 104.6158) (end 174.9446 104.6158) (width 0.25) (layer "B.Cu") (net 20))
 (segment (start 169.01 107.67) (end 170.3621 107.67) (width 0.25) (layer "F.Cu") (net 8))
 (via (at 170.3621 107.67) (size 0.8) (drill 0.4) (layers "F.Cu" "B.Cu") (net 8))
 (segment (start 180.2613 104.695) (end 181.8364 104.695) (width 0.25) (layer "B.Cu") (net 8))
 (segment (start 181.61 59.69) (end 181.61 60.8651) (width 0.25) (layer "B.Cu") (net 8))
 (segment (start 170.3621 107.67) (end 175.7112 107.67) (width 0.25) (layer "B.Cu") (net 8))
 (segment (start 183.3101 62.198) (end 181.9772 60.8651) (width 0.25) (layer "B.Cu") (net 8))
 (segment (start 181.8364 104.695) (end 183.3101 103.2213) (width 0.25) (layer "B.Cu") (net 8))
 (segment (start 180.2613 104.695) (end 178.6862 104.695) (width 0.25) (layer "B.Cu") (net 8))
 (segment (start 183.3101 103.2213) (end 183.3101 62.198) (width 0.25) (layer "B.Cu") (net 8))
 (segment (start 175.7112 107.67) (end 178.6862 104.695) (width 0.25) (layer "B.Cu") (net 8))
 (segment (start 181.9772 60.8651) (end 181.61 60.8651) (width 0.25) (layer "B.Cu") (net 8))
 (segment (start 168.9485 103.0585) (end 168.9485 102.2851) (width 0.25) (layer "F.Cu") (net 1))
 (segment (start 169.01 103.12) (end 168.9485 103.0585) (width 0.25) (layer "F.Cu") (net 1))
 (via (at 168.9485 102.2851) (size 0.8) (drill 0.4) (layers "F.Cu" "B.Cu") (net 1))
 (segment (start 168.9485 102.2851) (end 173.3998 102.2851) (width 0.25) (layer "B.Cu") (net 1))
 (segment (start 173.3998 102.2851) (end 180.4349 95.25) (width 0.25) (layer "B.Cu") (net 1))
 (segment (start 181.61 95.25) (end 180.4349 95.25) (width 0.25) (layer "B.Cu") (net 1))
 (segment (start 169.01 103.77) (end 168.2464 103.77) (width 0.25) (layer "F.Cu") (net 2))
 (segment (start 168.2464 103.77) (end 167.67 103.1936) (width 0.25) (layer "F.Cu") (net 2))
 (via (at 167.67 103.1936) (size 0.8) (drill 0.4) (layers "F.Cu" "B.Cu") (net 2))
 (segment (start 180.4349 97.79) (end 175.0313 103.1936) (width 0.25) (layer "B.Cu") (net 2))
 (segment (start 181.61 97.79) (end 180.4349 97.79) (width 0.25) (layer "B.Cu") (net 2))
 (segment (start 175.0313 103.1936) (end 167.67 103.1936) (width 0.25) (layer "B.Cu") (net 2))
 (segment (start 169.01 105.72) (end 168.2957 105.72) (width 0.25) (layer "F.Cu") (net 5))
 (segment (start 163.83 92.71) (end 165.0051 92.71) (width 0.25) (layer "F.Cu") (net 5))
 (segment (start 167.9276 105.3519) (end 167.9276 104.6483) (width 0.25) (layer "F.Cu") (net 5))
 (segment (start 165.0051 101.7258) (end 165.0051 92.71) (width 0.25) (layer "F.Cu") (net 5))
 (segment (start 168.2957 105.72) (end 167.9276 105.3519) (width 0.25) (layer "F.Cu") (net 5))
 (segment (start 167.9276 104.6483) (end 165.0051 101.7258) (width 0.25) (layer "F.Cu") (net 5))
 (segment (start 164.0338 108.5087) (end 160.8549 105.3298) (width 0.25) (layer "F.Cu") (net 11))
 (segment (start 168.3124 109.62) (end 167.7128 110.2196) (width 0.25) (layer "F.Cu") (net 11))
 (segment (start 167.7128 110.2196) (end 164.4423 110.2196) (width 0.25) (layer "F.Cu") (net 11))
 (segment (start 169.01 109.62) (end 168.3124 109.62) (width 0.25) (layer "F.Cu") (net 11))
 (segment (start 164.0338 109.8111) (end 164.0338 108.5087) (width 0.25) (layer "F.Cu") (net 11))
 (segment (start 164.4423 110.2196) (end 164.0338 109.8111) (width 0.25) (layer "F.Cu") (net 11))
 (segment (start 163.83 72.39) (end 160.8549 72.39) (width 0.25) (layer "F.Cu") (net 11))
 (segment (start 160.8549 105.3298) (end 160.8549 72.39) (width 0.25) (layer "F.Cu") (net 11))
 (segment (start 174.0456 108.97) (end 170.8568 105.7812) (width 0.25) (layer "F.Cu") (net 15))
 (segment (start 174.735 108.97) (end 174.0456 108.97) (width 0.25) (layer "F.Cu") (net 15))
 (segment (start 168.8224 101.4353) (end 168.1047 100.7176) (width 0.25) (layer "F.Cu") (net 15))
 (segment (start 169.1358 101.4353) (end 168.8224 101.4353) (width 0.25) (layer "F.Cu") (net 15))
 (segment (start 163.83 77.47) (end 165.0051 77.47) (width 0.25) (layer "F.Cu") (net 15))
 (segment (start 170.8568 103.1563) (end 169.1358 101.4353) (width 0.25) (layer "F.Cu") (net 15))
 (segment (start 168.1047 80.5696) (end 165.0051 77.47) (width 0.25) (layer "F.Cu") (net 15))
 (segment (start 170.8568 105.7812) (end 170.8568 103.1563) (width 0.25) (layer "F.Cu") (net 15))
 (segment (start 168.1047 100.7176) (end 168.1047 80.5696) (width 0.25) (layer "F.Cu") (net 15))
 (segment (start 174.0323 108.32) (end 171.3069 105.5946) (width 0.25) (layer "F.Cu") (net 16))
 (segment (start 168.5548 100.5311) (end 168.5548 78.4797) (width 0.25) (layer "F.Cu") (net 16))
 (segment (start 171.3069 102.9698) (end 169.3223 100.9852) (width 0.25) (layer "F.Cu") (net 16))
 (segment (start 168.5548 78.4797) (end 165.0051 74.93) (width 0.25) (layer "F.Cu") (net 16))
 (segment (start 174.735 108.32) (end 174.0323 108.32) (width 0.25) (layer "F.Cu") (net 16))
 (segment (start 169.0089 100.9852) (end 168.5548 100.5311) (width 0.25) (layer "F.Cu") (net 16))
 (segment (start 163.83 74.93) (end 165.0051 74.93) (width 0.25) (layer "F.Cu") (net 16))
 (segment (start 171.3069 105.5946) (end 171.3069 102.9698) (width 0.25) (layer "F.Cu") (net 16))
 (segment (start 169.3223 100.9852) (end 169.0089 100.9852) (width 0.25) (layer "F.Cu") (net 16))
 (segment (start 169.0049 100.3446) (end 169.0049 75.7961) (width 0.25) (layer "F.Cu") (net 17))
 (segment (start 174.0201 107.67) (end 171.757 105.4069) (width 0.25) (layer "F.Cu") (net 17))
 (segment (start 169.5671 100.5351) (end 169.1954 100.5351) (width 0.25) (layer "F.Cu") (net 17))
 (segment (start 171.757 105.4069) (end 171.757 102.725) (width 0.25) (layer "F.Cu") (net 17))
 (segment (start 163.83 69.85) (end 163.83 71.0251) (width 0.25) (layer "F.Cu") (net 17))
 (segment (start 174.735 107.67) (end 174.0201 107.67) (width 0.25) (layer "F.Cu") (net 17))
 (segment (start 171.757 102.725) (end 169.5671 100.5351) (width 0.25) (layer "F.Cu") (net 17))
 (segment (start 169.0049 75.7961) (end 164.2339 71.0251) (width 0.25) (layer "F.Cu") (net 17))
 (segment (start 164.2339 71.0251) (end 163.83 71.0251) (width 0.25) (layer "F.Cu") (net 17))
 (segment (start 169.1954 100.5351) (end 169.0049 100.3446) (width 0.25) (layer "F.Cu") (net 17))
 (segment (start 174.0068 107.02) (end 172.2484 105.2616) (width 0.25) (layer "F.Cu") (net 18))
 (segment (start 171.5228 100.4776) (end 171.5228 89.4734) (width 0.25) (layer "F.Cu") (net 18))
 (segment (start 172.2484 101.2032) (end 171.5228 100.4776) (width 0.25) (layer "F.Cu") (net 18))
 (segment (start 172.2484 105.2616) (end 172.2484 101.2032) (width 0.25) (layer "F.Cu") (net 18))
 (segment (start 174.735 107.02) (end 174.0068 107.02) (width 0.25) (layer "F.Cu") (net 18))
 (via (at 171.5228 89.4734) (size 0.8) (drill 0.4) (layers "F.Cu" "B.Cu") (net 18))
 (segment (start 171.5227 89.4734) (end 171.5228 89.4734) (width 0.25) (layer "B.Cu") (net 18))
 (segment (start 164.1972 81.1851) (end 171.5227 88.5106) (width 0.25) (layer "B.Cu") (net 18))
 (segment (start 163.83 80.01) (end 163.83 81.1851) (width 0.25) (layer "B.Cu") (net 18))
 (segment (start 163.83 81.1851) (end 164.1972 81.1851) (width 0.25) (layer "B.Cu") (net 18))
 (segment (start 171.5227 88.5106) (end 171.5227 89.4734) (width 0.25) (layer "B.Cu") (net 18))
 (segment (start 174.735 106.37) (end 174.0448 106.37) (width 0.25) (layer "F.Cu") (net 19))
 (segment (start 181.61 87.63) (end 181.61 88.8051) (width 0.25) (layer "F.Cu") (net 19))
 (segment (start 174.0448 106.37) (end 172.6986 105.0238) (width 0.25) (layer "F.Cu") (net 19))
 (segment (start 174.0849 100.7257) (end 174.0849 95.5223) (width 0.25) (layer "F.Cu") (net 19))
 (segment (start 172.6986 102.112) (end 174.0849 100.7257) (width 0.25) (layer "F.Cu") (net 19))
 (segment (start 174.0849 95.5223) (end 180.8021 88.8051) (width 0.25) (layer "F.Cu") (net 19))
 (segment (start 180.8021 88.8051) (end 181.61 88.8051) (width 0.25) (layer "F.Cu") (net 19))
 (segment (start 172.6986 105.0238) (end 172.6986 102.112) (width 0.25) (layer "F.Cu") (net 19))
 (segment (start 173.9737 105.07) (end 173.2004 104.2967) (width 0.25) (layer "F.Cu") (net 21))
 (segment (start 178.9017 97.8886) (end 178.9017 91.7032) (width 0.25) (layer "F.Cu") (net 21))
 (segment (start 173.2004 102.6602) (end 175.1898 100.6708) (width 0.25) (layer "F.Cu") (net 21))
 (segment (start 181.61 90.17) (end 180.4349 90.17) (width 0.25) (layer "F.Cu") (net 21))
 (segment (start 176.1195 100.6708) (end 178.9017 97.8886) (width 0.25) (layer "F.Cu") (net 21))
 (segment (start 175.1898 100.6708) (end 176.1195 100.6708) (width 0.25) (layer "F.Cu") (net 21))
 (segment (start 173.2004 104.2967) (end 173.2004 102.6602) (width 0.25) (layer "F.Cu") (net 21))
 (segment (start 178.9017 91.7032) (end 180.4349 90.17) (width 0.25) (layer "F.Cu") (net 21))
 (segment (start 174.735 105.07) (end 173.9737 105.07) (width 0.25) (layer "F.Cu") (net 21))
 (segment (start 176.0114 104.42) (end 176.1102 104.3212) (width 0.25) (layer "F.Cu") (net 22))
 (segment (start 174.735 104.42) (end 176.0114 104.42) (width 0.25) (layer "F.Cu") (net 22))
 (via (at 176.1102 104.3212) (size 0.8) (drill 0.4) (layers "F.Cu" "B.Cu") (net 22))
 (segment (start 178.9653 101.1698) (end 176.1102 104.0249) (width 0.25) (layer "B.Cu") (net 22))
 (segment (start 179.9041 101.1698) (end 178.9653 101.1698) (width 0.25) (layer "B.Cu") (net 22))
 (segment (start 181.61 86.2651) (end 181.9752 86.2651) (width 0.25) (layer "B.Cu") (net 22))
 (segment (start 182.8042 98.2697) (end 179.9041 101.1698) (width 0.25) (layer "B.Cu") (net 22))
 (segment (start 176.1102 104.0249) (end 176.1102 104.3212) (width 0.25) (layer "B.Cu") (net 22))
 (segment (start 182.8042 87.0941) (end 182.8042 98.2697) (width 0.25) (layer "B.Cu") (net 22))
 (segment (start 181.61 85.09) (end 181.61 86.2651) (width 0.25) (layer "B.Cu") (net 22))
 (segment (start 181.9752 86.2651) (end 182.8042 87.0941) (width 0.25) (layer "B.Cu") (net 22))
 (segment (start 174.0293 103.77) (end 173.6516 103.3923) (width 0.25) (layer "F.Cu") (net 23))
 (segment (start 180.4349 96.9938) (end 180.4349 94.2523) (width 0.25) (layer "F.Cu") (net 23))
 (segment (start 173.6516 102.8594) (end 173.9166 102.5944) (width 0.25) (layer "F.Cu") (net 23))
 (segment (start 181.61 92.71) (end 181.61 93.8851) (width 0.25) (layer "F.Cu") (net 23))
 (segment (start 174.8343 102.5944) (end 180.4349 96.9938) (width 0.25) (layer "F.Cu") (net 23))
 (segment (start 180.8021 93.8851) (end 181.61 93.8851) (width 0.25) (layer "F.Cu") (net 23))
 (segment (start 173.9166 102.5944) (end 174.8343 102.5944) (width 0.25) (layer "F.Cu") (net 23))
 (segment (start 174.735 103.77) (end 174.0293 103.77) (width 0.25) (layer "F.Cu") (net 23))
 (segment (start 180.4349 94.2523) (end 180.8021 93.8851) (width 0.25) (layer "F.Cu") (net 23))
 (segment (start 173.6516 103.3923) (end 173.6516 102.8594) (width 0.25) (layer "F.Cu") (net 23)))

